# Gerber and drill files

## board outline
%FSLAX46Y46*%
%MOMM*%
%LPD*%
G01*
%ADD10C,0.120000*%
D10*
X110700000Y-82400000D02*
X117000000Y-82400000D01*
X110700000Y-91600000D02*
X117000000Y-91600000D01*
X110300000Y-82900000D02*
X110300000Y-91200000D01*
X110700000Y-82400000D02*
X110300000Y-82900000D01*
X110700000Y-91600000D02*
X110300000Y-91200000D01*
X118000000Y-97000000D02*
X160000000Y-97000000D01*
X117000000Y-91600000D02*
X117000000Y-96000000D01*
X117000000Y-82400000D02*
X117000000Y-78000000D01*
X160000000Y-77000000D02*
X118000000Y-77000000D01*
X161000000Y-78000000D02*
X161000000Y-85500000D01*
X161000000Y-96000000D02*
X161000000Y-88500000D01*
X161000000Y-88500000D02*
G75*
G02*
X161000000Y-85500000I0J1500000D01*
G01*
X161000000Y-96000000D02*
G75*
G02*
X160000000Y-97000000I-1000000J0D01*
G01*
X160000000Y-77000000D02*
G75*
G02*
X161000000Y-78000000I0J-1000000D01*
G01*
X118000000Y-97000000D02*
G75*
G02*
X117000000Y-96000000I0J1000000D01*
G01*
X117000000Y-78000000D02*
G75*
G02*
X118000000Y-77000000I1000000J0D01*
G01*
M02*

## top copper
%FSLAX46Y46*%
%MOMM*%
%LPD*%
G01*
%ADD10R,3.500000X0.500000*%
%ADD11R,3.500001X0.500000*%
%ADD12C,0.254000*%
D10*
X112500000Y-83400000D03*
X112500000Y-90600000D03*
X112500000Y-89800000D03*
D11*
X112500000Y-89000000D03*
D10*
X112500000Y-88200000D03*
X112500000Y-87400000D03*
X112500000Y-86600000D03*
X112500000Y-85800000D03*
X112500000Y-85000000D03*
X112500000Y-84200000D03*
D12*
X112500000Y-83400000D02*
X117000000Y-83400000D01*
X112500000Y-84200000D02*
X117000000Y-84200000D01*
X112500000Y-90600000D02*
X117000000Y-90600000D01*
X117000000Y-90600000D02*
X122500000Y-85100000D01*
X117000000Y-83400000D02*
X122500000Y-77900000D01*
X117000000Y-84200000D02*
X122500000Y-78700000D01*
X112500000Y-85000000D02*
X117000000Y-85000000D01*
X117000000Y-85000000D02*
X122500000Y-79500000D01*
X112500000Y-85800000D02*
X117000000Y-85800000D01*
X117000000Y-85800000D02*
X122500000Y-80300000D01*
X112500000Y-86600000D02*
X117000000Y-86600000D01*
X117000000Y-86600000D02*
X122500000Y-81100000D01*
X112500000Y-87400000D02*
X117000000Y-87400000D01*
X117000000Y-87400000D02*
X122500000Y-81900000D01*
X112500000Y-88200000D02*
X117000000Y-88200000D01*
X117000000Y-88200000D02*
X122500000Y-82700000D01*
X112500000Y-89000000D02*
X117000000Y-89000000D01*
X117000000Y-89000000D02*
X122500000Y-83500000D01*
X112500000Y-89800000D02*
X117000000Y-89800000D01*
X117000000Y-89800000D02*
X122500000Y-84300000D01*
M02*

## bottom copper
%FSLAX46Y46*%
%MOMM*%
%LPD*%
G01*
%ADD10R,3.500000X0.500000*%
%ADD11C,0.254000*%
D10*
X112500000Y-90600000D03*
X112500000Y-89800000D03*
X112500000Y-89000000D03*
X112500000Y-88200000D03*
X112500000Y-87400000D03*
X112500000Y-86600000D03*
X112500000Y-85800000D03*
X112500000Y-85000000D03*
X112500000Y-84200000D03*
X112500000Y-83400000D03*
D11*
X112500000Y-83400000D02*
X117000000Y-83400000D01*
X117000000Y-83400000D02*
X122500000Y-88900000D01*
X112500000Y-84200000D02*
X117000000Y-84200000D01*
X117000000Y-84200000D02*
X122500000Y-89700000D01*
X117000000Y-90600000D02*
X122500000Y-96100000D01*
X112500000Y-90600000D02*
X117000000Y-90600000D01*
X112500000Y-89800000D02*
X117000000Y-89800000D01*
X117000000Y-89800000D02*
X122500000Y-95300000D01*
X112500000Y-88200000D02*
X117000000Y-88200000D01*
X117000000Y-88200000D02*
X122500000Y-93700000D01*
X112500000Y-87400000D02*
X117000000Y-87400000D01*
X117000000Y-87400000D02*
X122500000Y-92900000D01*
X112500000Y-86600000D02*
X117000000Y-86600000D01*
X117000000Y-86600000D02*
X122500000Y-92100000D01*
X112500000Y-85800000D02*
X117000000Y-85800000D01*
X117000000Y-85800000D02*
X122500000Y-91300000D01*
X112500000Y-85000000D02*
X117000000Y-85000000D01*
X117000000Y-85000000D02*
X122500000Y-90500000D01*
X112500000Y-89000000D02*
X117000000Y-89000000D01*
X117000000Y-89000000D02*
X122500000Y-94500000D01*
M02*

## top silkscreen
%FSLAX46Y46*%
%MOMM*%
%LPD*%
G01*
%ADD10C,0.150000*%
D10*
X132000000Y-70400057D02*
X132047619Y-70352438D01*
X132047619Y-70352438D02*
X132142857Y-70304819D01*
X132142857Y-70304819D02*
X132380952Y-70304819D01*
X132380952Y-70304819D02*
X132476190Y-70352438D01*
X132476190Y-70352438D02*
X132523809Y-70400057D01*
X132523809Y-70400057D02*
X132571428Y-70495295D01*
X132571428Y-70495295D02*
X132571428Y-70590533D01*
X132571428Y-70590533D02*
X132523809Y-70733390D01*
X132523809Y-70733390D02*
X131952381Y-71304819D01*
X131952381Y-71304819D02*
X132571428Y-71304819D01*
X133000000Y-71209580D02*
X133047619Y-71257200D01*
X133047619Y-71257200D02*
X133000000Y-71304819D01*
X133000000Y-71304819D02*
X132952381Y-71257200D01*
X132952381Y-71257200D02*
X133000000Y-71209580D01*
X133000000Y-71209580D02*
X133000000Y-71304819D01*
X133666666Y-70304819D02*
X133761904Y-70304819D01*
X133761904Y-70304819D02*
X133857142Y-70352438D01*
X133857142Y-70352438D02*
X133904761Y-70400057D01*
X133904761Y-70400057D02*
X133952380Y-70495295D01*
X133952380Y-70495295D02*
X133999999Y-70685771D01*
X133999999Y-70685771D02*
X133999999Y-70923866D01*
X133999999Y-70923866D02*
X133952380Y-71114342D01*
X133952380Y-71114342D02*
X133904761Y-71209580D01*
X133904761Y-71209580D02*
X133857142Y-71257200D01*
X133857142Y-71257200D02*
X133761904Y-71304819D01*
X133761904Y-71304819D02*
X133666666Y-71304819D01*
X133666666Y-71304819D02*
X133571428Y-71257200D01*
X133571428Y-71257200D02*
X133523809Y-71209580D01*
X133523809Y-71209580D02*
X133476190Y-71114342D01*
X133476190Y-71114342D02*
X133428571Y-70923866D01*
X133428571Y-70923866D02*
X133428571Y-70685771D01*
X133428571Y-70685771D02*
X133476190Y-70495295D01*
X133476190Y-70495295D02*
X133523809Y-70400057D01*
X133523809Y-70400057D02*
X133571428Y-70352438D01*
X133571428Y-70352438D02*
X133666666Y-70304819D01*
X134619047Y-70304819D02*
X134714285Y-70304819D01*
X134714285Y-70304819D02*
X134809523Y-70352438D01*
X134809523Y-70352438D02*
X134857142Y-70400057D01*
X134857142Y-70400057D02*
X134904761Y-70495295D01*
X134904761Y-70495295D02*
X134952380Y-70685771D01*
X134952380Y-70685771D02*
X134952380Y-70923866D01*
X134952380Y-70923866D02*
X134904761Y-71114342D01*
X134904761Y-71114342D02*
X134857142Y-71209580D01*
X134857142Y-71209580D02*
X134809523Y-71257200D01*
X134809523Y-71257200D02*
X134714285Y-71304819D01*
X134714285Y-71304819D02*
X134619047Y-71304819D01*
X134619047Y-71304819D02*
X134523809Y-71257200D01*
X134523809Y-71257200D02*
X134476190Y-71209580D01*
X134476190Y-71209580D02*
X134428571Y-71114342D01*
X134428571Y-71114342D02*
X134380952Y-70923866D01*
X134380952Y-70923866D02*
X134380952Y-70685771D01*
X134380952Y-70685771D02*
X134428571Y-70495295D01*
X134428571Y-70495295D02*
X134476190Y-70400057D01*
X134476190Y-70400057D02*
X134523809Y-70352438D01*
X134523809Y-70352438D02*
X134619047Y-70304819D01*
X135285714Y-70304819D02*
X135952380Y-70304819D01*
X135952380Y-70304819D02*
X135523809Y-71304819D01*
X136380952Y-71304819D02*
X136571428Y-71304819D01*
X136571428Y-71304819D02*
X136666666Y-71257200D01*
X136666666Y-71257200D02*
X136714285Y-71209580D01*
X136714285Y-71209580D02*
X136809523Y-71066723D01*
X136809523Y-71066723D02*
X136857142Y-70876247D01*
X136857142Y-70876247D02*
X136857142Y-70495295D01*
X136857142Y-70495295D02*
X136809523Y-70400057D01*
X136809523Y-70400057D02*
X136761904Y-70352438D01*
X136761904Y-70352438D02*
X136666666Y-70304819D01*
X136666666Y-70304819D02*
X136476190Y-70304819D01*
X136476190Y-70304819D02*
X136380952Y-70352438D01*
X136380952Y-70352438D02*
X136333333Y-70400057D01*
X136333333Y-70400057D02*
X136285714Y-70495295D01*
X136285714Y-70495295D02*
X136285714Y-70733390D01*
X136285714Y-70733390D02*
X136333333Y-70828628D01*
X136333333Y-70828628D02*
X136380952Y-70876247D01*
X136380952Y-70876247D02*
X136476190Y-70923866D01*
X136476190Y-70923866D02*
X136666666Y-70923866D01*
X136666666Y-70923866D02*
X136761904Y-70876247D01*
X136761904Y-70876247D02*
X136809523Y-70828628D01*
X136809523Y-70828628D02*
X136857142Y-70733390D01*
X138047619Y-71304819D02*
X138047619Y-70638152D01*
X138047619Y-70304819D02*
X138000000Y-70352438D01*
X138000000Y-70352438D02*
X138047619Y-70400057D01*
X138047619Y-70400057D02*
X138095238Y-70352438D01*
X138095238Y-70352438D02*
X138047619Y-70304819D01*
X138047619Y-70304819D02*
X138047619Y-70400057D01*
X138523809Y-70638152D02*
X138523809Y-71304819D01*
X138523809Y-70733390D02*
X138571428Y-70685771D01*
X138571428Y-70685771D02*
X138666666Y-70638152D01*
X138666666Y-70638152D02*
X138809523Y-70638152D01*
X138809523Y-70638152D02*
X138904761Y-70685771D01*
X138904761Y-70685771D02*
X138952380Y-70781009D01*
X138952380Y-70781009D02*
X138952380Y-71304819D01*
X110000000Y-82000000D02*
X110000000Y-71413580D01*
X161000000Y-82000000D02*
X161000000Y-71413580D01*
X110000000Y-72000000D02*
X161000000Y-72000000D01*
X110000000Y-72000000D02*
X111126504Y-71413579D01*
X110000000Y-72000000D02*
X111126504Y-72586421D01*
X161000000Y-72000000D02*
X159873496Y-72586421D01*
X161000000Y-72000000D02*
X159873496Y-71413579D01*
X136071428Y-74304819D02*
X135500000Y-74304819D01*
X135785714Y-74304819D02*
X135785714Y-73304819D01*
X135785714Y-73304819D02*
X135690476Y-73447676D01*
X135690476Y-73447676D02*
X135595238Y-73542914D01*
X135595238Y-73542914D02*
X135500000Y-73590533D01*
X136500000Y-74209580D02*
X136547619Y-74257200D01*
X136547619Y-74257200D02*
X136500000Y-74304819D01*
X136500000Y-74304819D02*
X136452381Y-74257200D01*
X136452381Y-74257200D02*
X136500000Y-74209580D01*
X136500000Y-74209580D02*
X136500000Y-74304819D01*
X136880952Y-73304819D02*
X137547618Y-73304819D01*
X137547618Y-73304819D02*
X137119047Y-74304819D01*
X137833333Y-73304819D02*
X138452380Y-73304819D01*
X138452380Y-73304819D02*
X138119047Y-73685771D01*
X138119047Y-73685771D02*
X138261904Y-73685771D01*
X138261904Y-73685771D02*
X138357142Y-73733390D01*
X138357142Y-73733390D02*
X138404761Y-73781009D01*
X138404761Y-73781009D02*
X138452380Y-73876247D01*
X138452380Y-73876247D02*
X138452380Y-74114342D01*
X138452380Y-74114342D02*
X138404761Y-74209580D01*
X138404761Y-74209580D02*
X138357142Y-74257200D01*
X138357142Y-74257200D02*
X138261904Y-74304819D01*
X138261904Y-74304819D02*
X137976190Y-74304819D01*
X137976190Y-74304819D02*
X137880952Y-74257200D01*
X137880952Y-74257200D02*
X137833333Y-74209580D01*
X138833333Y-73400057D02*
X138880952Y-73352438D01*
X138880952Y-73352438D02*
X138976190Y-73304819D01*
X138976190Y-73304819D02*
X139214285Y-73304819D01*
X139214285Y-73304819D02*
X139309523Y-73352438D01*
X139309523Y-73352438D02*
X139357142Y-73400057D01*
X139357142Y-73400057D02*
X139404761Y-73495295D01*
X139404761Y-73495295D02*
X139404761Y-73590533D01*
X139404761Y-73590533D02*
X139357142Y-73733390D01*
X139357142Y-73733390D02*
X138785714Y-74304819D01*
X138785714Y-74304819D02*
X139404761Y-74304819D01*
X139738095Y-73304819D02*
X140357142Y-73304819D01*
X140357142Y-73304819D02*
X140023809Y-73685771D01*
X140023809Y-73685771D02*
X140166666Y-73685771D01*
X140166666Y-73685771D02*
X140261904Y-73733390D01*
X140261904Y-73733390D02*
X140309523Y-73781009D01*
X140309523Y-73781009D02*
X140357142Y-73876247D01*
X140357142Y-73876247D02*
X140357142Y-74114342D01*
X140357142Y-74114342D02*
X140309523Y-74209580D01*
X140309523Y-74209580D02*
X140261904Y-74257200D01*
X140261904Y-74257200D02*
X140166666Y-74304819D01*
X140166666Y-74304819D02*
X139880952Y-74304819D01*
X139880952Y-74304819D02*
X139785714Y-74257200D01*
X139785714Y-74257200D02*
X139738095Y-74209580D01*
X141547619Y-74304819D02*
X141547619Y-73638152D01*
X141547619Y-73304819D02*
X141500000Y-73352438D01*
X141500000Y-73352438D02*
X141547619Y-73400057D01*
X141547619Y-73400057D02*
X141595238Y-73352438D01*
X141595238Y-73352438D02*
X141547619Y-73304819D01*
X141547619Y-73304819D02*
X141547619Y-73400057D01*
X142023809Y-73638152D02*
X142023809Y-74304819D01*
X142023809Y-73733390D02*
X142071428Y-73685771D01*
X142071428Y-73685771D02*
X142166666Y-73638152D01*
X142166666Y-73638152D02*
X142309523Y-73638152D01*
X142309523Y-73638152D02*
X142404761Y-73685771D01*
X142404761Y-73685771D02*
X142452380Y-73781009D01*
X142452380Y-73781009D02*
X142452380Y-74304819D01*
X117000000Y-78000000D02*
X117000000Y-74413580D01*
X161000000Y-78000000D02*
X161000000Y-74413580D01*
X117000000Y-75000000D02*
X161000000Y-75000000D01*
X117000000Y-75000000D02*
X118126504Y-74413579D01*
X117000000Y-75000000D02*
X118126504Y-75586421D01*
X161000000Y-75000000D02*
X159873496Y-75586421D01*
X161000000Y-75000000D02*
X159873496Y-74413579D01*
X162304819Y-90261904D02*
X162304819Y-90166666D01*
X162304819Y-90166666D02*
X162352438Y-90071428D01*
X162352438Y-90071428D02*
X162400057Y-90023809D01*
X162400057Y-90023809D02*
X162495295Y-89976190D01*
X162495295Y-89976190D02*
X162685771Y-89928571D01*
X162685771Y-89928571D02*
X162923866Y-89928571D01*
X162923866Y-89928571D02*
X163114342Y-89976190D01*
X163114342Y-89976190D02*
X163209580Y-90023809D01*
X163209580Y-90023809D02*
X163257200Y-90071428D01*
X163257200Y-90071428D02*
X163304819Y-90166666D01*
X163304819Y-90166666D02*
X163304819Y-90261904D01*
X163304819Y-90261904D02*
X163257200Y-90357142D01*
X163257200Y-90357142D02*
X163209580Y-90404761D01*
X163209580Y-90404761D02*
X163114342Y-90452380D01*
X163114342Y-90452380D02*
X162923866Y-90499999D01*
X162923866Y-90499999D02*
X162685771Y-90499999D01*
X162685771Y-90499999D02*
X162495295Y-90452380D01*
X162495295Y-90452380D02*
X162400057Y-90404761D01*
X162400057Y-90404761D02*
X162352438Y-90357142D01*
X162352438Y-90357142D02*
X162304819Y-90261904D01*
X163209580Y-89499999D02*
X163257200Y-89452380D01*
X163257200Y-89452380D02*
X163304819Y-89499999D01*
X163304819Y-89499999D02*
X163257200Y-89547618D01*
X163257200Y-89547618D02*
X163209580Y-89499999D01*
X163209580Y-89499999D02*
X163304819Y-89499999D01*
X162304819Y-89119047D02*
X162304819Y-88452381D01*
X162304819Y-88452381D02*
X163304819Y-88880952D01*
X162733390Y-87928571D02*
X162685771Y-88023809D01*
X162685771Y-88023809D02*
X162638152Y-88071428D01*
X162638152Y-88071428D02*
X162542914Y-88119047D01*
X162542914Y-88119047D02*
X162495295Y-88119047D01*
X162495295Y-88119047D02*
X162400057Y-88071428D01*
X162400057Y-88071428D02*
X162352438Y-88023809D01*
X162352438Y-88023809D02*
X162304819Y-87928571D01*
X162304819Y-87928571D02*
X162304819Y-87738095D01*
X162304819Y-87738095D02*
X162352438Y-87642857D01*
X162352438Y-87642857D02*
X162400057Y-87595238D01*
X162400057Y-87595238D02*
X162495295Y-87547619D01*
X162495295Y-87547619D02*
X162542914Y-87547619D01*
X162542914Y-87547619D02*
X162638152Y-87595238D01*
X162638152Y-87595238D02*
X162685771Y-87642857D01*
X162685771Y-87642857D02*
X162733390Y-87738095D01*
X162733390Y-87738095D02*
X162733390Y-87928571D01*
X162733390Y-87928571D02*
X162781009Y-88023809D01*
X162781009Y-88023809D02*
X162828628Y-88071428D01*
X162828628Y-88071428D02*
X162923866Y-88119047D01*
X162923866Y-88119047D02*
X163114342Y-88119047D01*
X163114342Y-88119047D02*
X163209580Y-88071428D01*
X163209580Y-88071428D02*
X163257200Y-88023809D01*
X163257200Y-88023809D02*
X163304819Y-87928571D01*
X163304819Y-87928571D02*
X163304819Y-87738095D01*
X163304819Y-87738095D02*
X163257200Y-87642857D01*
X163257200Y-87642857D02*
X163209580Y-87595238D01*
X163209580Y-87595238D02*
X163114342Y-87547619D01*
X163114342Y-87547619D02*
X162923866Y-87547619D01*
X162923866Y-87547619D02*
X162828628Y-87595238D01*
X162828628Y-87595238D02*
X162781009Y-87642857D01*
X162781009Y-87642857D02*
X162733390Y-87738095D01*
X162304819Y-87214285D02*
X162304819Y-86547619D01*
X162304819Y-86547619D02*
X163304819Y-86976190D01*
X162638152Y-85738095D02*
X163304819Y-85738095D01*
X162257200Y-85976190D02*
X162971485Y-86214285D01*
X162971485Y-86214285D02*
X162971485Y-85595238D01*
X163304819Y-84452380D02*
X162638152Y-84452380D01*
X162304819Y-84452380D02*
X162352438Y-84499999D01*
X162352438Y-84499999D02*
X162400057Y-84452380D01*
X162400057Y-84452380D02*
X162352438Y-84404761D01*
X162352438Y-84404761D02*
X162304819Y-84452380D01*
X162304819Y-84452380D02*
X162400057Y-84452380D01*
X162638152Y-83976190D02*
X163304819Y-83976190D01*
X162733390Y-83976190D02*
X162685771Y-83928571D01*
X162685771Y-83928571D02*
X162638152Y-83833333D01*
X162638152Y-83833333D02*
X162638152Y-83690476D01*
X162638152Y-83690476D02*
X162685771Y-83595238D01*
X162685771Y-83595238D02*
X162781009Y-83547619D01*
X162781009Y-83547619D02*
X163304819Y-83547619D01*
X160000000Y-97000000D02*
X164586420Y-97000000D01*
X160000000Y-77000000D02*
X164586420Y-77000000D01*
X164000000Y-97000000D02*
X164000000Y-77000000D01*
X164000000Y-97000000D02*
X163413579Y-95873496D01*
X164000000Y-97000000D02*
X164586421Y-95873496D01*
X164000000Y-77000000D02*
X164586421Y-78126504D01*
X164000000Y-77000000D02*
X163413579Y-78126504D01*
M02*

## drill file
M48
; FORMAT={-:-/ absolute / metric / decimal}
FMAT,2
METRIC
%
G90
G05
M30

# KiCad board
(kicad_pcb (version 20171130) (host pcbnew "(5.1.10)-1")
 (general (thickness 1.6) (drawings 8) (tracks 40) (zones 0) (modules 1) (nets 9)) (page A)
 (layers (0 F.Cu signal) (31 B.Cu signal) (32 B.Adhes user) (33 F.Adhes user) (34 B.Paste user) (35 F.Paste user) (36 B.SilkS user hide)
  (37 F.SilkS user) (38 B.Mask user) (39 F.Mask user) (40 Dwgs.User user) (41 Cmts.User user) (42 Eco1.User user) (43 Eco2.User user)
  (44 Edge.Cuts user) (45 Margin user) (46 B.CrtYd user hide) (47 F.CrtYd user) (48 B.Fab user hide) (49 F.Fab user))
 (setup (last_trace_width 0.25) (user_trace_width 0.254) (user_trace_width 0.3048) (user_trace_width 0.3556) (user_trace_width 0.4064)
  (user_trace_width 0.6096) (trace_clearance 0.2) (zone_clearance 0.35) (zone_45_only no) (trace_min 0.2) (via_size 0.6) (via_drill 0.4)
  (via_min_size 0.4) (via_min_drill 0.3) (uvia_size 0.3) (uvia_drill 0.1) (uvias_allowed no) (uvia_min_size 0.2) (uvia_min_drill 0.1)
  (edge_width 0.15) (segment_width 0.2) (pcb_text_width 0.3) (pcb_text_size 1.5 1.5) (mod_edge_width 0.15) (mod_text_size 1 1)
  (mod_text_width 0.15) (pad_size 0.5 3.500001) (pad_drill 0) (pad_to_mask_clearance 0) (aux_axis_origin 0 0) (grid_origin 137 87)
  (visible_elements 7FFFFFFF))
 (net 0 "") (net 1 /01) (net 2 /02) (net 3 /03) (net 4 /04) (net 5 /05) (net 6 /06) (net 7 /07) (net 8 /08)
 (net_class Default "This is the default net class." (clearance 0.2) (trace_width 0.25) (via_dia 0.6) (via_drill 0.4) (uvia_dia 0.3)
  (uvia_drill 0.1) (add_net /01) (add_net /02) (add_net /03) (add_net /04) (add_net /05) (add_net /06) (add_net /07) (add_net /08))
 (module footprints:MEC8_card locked (layer F.Cu) (at 112.5 87 90)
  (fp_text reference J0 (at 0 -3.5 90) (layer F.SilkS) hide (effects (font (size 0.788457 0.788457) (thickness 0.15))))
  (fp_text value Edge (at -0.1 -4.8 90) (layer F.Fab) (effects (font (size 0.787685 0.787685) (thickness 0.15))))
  (fp_line (start 4.6 -1.8) (end 4.6 4.5) (layer Edge.Cuts) (width 0.12))
  (fp_line (start -4.6 -1.8) (end -4.6 4.5) (layer Edge.Cuts) (width 0.12))
  (fp_line (start 4.1 -2.2) (end -4.2 -2.2) (layer Edge.Cuts) (width 0.12))
  (fp_line (start 4.6 -1.8) (end 4.1 -2.2) (layer Edge.Cuts) (width 0.12))
  (fp_line (start -4.6 -1.8) (end -4.2 -2.2) (layer Edge.Cuts) (width 0.12))
  (fp_line (start -10 5.5) (end -10 47.5) (layer Edge.Cuts) (width 0.12))
  (fp_line (start -4.6 4.5) (end -9 4.5) (layer Edge.Cuts) (width 0.12))
  (fp_line (start 4.6 4.5) (end 9 4.5) (layer Edge.Cuts) (width 0.12))
  (fp_line (start 10 47.5) (end 10 5.5) (layer Edge.Cuts) (width 0.12))
  (fp_line (start 9 48.5) (end 1.5 48.5) (layer Edge.Cuts) (width 0.12))
  (fp_line (start -9 48.5) (end -1.5 48.5) (layer Edge.Cuts) (width 0.12))
  (fp_arc (start 0 48.5) (end 1.5 48.5) (angle -180) (layer Edge.Cuts) (width 0.12))
  (fp_arc (start -9 47.5) (end -10 47.5) (angle -90) (layer Edge.Cuts) (width 0.12))
  (fp_arc (start 9 47.5) (end 9 48.5) (angle -90) (layer Edge.Cuts) (width 0.12))
  (fp_arc (start -9 5.5) (end -9 4.5) (angle -90) (layer Edge.Cuts) (width 0.12))
  (fp_arc (start 9 5.5) (end 10 5.5) (angle -90) (layer Edge.Cuts) (width 0.12))
  (pad 20 smd rect (at 3.6 0 90) (size 0.5 3.5) (layers F.Cu F.Paste F.Mask))
  (pad 11 smd rect (at -3.6 0 90) (size 0.5 3.5) (layers F.Cu F.Paste F.Mask))
  (pad 12 smd rect (at -2.8 0 90) (size 0.5 3.5) (layers F.Cu F.Paste F.Mask))
  (pad 13 smd rect (at -2 0 90) (size 0.5 3.500001) (layers F.Cu F.Paste F.Mask))
  (pad 14 smd rect (at -1.2 0 90) (size 0.5 3.5) (layers F.Cu F.Paste F.Mask))
  (pad 15 smd rect (at -0.4 0 90) (size 0.5 3.5) (layers F.Cu F.Paste F.Mask))
  (pad 16 smd rect (at 0.4 0 90) (size 0.5 3.5) (layers F.Cu F.Paste F.Mask))
  (pad 17 smd rect (at 1.2 0 90) (size 0.5 3.5) (layers F.Cu F.Paste F.Mask))
  (pad 18 smd rect (at 2 0 90) (size 0.5 3.5) (layers F.Cu F.Paste F.Mask))
  (pad 19 smd rect (at 2.8 0 90) (size 0.5 3.5) (layers F.Cu F.Paste F.Mask))
  (pad 1 smd rect (at -3.6 0 90) (size 0.5 3.5) (layers B.Cu B.Paste B.Mask) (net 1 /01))
  (pad 2 smd rect (at -2.8 0 90) (size 0.5 3.5) (layers B.Cu B.Paste B.Mask) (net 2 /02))
  (pad 3 smd rect (at -2 0 90) (size 0.5 3.5) (layers B.Cu B.Paste B.Mask) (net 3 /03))
  (pad 4 smd rect (at -1.2 0 90) (size 0.5 3.5) (layers B.Cu B.Paste B.Mask) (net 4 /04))
  (pad 5 smd rect (at -0.4 0 90) (size 0.5 3.5) (layers B.Cu B.Paste B.Mask) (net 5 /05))
  (pad 6 smd rect (at 0.4 0 90) (size 0.5 3.5) (layers B.Cu B.Paste B.Mask) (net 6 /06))
  (pad 7 smd rect (at 1.2 0 90) (size 0.5 3.5) (layers B.Cu B.Paste B.Mask) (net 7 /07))
  (pad 8 smd rect (at 2 0 90) (size 0.5 3.5) (layers B.Cu B.Paste B.Mask) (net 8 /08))
  (pad 9 smd rect (at 2.8 0 90) (size 0.5 3.5) (layers B.Cu B.Paste B.Mask))
  (pad 10 smd rect (at 3.6 0 90) (size 0.5 3.5) (layers B.Cu B.Paste B.Mask)))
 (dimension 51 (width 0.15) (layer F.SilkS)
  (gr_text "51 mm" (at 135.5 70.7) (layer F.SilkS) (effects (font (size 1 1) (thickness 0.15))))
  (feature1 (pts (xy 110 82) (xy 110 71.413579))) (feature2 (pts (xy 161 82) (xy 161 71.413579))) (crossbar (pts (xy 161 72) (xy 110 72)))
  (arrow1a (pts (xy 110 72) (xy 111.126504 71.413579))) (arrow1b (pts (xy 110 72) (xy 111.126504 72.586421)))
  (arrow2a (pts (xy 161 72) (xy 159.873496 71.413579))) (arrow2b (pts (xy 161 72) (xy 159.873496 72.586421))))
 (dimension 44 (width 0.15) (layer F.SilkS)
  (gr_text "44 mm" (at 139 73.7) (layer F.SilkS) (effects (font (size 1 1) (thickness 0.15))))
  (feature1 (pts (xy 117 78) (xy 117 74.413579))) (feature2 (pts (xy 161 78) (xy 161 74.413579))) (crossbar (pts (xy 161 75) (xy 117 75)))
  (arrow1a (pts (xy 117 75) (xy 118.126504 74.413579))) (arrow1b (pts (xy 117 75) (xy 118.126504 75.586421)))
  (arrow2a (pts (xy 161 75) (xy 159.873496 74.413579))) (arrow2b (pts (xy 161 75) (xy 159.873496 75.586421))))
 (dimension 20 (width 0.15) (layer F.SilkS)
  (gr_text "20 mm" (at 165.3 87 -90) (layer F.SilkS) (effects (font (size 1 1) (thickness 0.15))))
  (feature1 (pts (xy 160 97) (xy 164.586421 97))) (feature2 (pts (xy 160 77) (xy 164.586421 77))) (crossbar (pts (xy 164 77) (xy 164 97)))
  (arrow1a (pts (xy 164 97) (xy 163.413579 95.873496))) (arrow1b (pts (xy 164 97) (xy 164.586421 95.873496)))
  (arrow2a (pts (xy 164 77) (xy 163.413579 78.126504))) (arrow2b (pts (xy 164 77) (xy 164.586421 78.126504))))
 (segment (start 112.5 83.4) (end 117 83.4) (width 0.254) (layer F.Cu) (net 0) (status 10))
 (segment (start 112.5 84.2) (end 117 84.2) (width 0.254) (layer F.Cu) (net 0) (status 10))
 (segment (start 112.5 90.6) (end 117 90.6) (width 0.254) (layer F.Cu) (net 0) (status 10))
 (segment (start 117 90.6) (end 122.5 85.1) (width 0.254) (layer F.Cu) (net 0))
 (segment (start 117 83.4) (end 122.5 77.9) (width 0.254) (layer F.Cu) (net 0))
 (segment (start 117 84.2) (end 122.5 78.7) (width 0.254) (layer F.Cu) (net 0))
 (segment (start 112.5 83.4) (end 117 83.4) (width 0.254) (layer B.Cu) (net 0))
 (segment (start 117 83.4) (end 122.5 88.9) (width 0.254) (layer B.Cu) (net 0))
 (segment (start 112.5 85) (end 117 85) (width 0.254) (layer F.Cu) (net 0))
 (segment (start 117 85) (end 122.5 79.5) (width 0.254) (layer F.Cu) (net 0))
 (segment (start 112.5 85.8) (end 117 85.8) (width 0.254) (layer F.Cu) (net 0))
 (segment (start 117 85.8) (end 122.5 80.3) (width 0.254) (layer F.Cu) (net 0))
 (segment (start 112.5 86.6) (end 117 86.6) (width 0.254) (layer F.Cu) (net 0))
 (segment (start 117 86.6) (end 122.5 81.1) (width 0.254) (layer F.Cu) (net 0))
 (segment (start 112.5 87.4) (end 117 87.4) (width 0.254) (layer F.Cu) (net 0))
 (segment (start 117 87.4) (end 122.5 81.9) (width 0.254) (layer F.Cu) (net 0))
 (segment (start 112.5 88.2) (end 117 88.2) (width 0.254) (layer F.Cu) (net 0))
 (segment (start 117 88.2) (end 122.5 82.7) (width 0.254) (layer F.Cu) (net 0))
 (segment (start 112.5 89) (end 117 89) (width 0.254) (layer F.Cu) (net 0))
 (segment (start 117 89) (end 122.5 83.5) (width 0.254) (layer F.Cu) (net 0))
 (segment (start 112.5 89.8) (end 117 89.8) (width 0.254) (layer F.Cu) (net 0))
 (segment (start 117 89.8) (end 122.5 84.3) (width 0.254) (layer F.Cu) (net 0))
 (segment (start 112.5 84.2) (end 117 84.2) (width 0.254) (layer B.Cu) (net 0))
 (segment (start 117 84.2) (end 122.5 89.7) (width 0.254) (layer B.Cu) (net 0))
 (segment (start 117 90.6) (end 122.5 96.1) (width 0.254) (layer B.Cu) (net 1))
 (segment (start 112.5 90.6) (end 117 90.6) (width 0.254) (layer B.Cu) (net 1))
 (segment (start 112.5 89.8) (end 117 89.8) (width 0.254) (layer B.Cu) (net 2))
 (segment (start 117 89.8) (end 122.5 95.3) (width 0.254) (layer B.Cu) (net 2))
 (segment (start 112.5 88.2) (end 117 88.2) (width 0.254) (layer B.Cu) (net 4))
 (segment (start 117 88.2) (end 122.5 93.7) (width 0.254) (layer B.Cu) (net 4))
 (segment (start 112.5 87.4) (end 117 87.4) (width 0.254) (layer B.Cu) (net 5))
 (segment (start 117 87.4) (end 122.5 92.9) (width 0.254) (layer B.Cu) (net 5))
 (segment (start 112.5 86.6) (end 117 86.6) (width 0.254) (layer B.Cu) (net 6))
 (segment (start 117 86.6) (end 122.5 92.1) (width 0.254) (layer B.Cu) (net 6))
 (segment (start 112.5 85.8) (end 117 85.8) (width 0.254) (layer B.Cu) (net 7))
 (segment (start 117 85.8) (end 122.5 91.3) (width 0.254) (layer B.Cu) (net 7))
 (segment (start 112.5 85) (end 117 85) (width 0.254) (layer B.Cu) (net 8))
 (segment (start 117 85) (end 122.5 90.5) (width 0.254) (layer B.Cu) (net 8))
 (segment (start 112.5 89) (end 117 89) (width 0.254) (layer B.Cu) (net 3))
 (segment (start 117 89) (end 122.5 94.5) (width 0.254) (layer B.Cu) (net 3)))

